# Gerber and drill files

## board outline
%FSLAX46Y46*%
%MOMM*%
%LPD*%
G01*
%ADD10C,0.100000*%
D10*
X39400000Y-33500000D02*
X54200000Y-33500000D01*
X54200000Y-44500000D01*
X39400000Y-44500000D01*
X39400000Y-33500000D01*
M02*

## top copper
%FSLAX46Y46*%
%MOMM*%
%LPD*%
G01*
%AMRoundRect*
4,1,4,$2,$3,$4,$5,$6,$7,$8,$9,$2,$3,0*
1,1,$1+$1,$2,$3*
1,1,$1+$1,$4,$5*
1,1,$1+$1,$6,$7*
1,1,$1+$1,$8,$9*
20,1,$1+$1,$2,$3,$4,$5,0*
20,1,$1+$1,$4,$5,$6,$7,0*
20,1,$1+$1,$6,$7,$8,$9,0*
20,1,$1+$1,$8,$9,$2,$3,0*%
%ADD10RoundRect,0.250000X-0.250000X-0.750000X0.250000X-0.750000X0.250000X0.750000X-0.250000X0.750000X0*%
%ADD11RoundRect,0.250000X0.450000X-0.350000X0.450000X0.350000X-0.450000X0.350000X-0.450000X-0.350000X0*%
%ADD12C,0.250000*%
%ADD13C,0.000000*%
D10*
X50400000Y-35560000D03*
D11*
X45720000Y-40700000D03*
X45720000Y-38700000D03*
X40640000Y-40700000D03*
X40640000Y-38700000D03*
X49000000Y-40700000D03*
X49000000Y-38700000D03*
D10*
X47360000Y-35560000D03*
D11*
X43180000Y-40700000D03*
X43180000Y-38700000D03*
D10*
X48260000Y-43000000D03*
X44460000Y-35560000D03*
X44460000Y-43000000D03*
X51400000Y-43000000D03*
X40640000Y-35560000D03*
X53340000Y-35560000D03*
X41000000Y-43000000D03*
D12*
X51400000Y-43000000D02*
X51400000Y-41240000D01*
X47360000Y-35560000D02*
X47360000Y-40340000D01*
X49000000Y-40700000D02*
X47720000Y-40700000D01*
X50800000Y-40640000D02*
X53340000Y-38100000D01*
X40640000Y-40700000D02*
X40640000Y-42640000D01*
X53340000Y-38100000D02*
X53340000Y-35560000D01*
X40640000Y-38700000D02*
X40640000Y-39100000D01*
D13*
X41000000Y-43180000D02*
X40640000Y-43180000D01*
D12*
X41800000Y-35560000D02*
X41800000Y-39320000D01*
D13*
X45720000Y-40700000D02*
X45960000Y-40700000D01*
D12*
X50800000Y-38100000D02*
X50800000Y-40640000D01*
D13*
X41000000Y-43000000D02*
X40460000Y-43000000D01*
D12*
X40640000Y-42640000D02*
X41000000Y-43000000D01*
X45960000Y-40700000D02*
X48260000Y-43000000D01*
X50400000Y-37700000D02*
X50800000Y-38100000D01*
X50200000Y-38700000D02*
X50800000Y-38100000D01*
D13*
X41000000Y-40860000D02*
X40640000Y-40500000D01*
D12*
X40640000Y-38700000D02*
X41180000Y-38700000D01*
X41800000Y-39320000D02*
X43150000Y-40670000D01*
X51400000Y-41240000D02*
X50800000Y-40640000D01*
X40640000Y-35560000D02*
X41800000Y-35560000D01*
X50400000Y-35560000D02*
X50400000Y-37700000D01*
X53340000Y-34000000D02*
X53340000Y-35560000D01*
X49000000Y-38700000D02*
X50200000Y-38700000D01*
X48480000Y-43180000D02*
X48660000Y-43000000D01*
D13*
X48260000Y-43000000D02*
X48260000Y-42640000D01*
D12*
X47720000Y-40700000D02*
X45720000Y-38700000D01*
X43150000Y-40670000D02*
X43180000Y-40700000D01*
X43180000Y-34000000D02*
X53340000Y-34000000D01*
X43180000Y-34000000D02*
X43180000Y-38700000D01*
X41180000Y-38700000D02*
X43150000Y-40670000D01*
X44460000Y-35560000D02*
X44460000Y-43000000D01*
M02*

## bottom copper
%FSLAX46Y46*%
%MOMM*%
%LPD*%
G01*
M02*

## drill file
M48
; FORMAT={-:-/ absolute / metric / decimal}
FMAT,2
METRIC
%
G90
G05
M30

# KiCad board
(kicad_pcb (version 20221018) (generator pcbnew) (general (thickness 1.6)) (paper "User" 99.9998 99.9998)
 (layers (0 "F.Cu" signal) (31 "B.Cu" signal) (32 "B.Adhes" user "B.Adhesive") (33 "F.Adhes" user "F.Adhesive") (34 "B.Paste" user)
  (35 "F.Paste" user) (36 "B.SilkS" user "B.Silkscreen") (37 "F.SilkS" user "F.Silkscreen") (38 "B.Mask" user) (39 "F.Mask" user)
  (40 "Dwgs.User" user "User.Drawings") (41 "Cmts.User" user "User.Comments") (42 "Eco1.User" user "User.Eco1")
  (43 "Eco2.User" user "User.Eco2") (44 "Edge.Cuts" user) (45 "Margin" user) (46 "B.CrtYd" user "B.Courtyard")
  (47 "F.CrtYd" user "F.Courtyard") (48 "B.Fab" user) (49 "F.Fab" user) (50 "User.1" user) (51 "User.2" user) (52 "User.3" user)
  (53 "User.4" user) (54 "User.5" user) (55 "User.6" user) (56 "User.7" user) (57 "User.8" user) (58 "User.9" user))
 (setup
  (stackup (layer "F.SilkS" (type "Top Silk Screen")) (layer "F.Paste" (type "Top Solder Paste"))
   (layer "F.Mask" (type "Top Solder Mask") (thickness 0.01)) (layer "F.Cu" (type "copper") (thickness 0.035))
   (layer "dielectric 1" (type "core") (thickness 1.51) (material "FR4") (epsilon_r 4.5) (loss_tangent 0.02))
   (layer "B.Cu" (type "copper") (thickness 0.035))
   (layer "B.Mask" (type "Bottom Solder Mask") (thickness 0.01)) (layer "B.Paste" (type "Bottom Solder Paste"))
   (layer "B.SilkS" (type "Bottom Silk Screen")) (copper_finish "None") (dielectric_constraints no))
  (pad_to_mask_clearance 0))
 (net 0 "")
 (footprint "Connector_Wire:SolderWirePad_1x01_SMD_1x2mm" (layer "F.Cu") (at 50.4 35.56)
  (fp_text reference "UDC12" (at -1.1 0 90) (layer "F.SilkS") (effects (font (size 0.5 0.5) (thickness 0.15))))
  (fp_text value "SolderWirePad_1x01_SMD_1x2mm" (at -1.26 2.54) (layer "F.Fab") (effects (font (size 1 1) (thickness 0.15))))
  (pad "1" smd roundrect (at 0 0) (size 1 2) (layers "F.Cu" "F.Paste" "F.Mask") (roundrect_rratio 0.25)))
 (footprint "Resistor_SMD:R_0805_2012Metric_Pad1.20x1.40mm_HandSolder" (layer "F.Cu") (at 45.72 39.7 90)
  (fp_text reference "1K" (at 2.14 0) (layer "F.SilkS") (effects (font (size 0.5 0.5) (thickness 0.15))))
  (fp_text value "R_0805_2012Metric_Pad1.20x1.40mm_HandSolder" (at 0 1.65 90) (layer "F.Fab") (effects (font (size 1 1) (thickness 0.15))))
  (pad "1" smd roundrect (at -1 0 90) (size 1.2 1.4) (layers "F.Cu" "F.Paste" "F.Mask") (roundrect_rratio 0.2083333333))
  (pad "2" smd roundrect (at 1 0 90) (size 1.2 1.4) (layers "F.Cu" "F.Paste" "F.Mask") (roundrect_rratio 0.2083333333)))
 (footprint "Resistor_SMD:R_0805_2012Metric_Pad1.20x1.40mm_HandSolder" (layer "F.Cu") (at 40.64 39.7 90)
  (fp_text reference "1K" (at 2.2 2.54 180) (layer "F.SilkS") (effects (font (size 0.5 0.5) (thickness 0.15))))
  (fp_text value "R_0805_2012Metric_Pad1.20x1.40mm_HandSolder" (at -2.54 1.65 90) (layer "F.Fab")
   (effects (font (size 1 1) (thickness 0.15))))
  (pad "1" smd roundrect (at -1 0 90) (size 1.2 1.4) (layers "F.Cu" "F.Paste" "F.Mask") (roundrect_rratio 0.2083333333))
  (pad "2" smd roundrect (at 1 0 90) (size 1.2 1.4) (layers "F.Cu" "F.Paste" "F.Mask") (roundrect_rratio 0.2083333333)))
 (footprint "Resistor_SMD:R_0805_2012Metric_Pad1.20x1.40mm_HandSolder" (layer "F.Cu") (at 49 39.7 90)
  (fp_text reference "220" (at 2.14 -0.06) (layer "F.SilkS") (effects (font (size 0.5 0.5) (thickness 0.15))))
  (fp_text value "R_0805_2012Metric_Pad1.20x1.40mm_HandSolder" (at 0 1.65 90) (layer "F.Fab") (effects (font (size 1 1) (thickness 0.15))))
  (pad "1" smd roundrect (at -1 0 90) (size 1.2 1.4) (layers "F.Cu" "F.Paste" "F.Mask") (roundrect_rratio 0.2083333333))
  (pad "2" smd roundrect (at 1 0 90) (size 1.2 1.4) (layers "F.Cu" "F.Paste" "F.Mask") (roundrect_rratio 0.2083333333)))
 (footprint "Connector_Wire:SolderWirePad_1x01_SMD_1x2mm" (layer "F.Cu") (at 47.36 35.56)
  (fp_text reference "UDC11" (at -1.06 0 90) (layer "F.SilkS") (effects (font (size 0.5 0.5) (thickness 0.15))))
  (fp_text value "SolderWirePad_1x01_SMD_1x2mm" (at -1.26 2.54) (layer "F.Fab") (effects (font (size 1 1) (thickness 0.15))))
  (pad "1" smd roundrect (at 0 0) (size 1 2) (layers "F.Cu" "F.Paste" "F.Mask") (roundrect_rratio 0.25)))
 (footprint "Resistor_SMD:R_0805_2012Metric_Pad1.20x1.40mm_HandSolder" (layer "F.Cu") (at 43.18 39.7 90)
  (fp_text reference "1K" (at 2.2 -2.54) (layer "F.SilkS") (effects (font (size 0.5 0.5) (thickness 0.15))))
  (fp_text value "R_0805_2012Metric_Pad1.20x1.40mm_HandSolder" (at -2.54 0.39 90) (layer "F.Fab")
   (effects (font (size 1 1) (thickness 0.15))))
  (pad "1" smd roundrect (at -1 0 90) (size 1.2 1.4) (layers "F.Cu" "F.Paste" "F.Mask") (roundrect_rratio 0.2083333333))
  (pad "2" smd roundrect (at 1 0 90) (size 1.2 1.4) (layers "F.Cu" "F.Paste" "F.Mask") (roundrect_rratio 0.2083333333)))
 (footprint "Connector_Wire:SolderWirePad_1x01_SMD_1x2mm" (layer "F.Cu") (at 48.26 43)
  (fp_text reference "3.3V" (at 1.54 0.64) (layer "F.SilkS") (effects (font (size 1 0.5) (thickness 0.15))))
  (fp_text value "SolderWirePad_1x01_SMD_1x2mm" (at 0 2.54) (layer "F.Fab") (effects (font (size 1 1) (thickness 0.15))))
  (pad "1" smd roundrect (at 0 0) (size 1 2) (layers "F.Cu" "F.Paste" "F.Mask") (roundrect_rratio 0.25)))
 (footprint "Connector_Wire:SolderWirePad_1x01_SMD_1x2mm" (layer "F.Cu") (at 44.46 35.56)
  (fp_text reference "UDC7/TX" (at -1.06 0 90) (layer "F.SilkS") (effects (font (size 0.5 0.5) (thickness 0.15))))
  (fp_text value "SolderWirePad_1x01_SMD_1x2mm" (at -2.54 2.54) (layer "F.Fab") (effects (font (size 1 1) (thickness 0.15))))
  (pad "1" smd roundrect (at 0 0) (size 1 2) (layers "F.Cu" "F.Paste" "F.Mask") (roundrect_rratio 0.25)))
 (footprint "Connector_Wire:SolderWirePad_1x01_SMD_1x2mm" (layer "F.Cu") (at 44.46 43)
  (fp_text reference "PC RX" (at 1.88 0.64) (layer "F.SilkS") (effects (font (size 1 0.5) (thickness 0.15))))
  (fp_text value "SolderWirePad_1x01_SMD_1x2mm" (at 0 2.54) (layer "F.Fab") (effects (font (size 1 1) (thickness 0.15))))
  (pad "1" smd roundrect (at 0 0) (size 1 2) (layers "F.Cu" "F.Paste" "F.Mask") (roundrect_rratio 0.25)))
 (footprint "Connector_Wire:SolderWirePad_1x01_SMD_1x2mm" (layer "F.Cu") (at 51.4 43)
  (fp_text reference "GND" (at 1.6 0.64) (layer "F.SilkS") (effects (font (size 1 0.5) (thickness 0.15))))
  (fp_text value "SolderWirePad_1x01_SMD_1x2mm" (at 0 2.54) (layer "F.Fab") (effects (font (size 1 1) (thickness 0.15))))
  (pad "1" smd roundrect (at 0 0) (size 1 2) (layers "F.Cu" "F.Paste" "F.Mask") (roundrect_rratio 0.25)))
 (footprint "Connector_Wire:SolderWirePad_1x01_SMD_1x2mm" (layer "F.Cu") (at 40.64 35.56)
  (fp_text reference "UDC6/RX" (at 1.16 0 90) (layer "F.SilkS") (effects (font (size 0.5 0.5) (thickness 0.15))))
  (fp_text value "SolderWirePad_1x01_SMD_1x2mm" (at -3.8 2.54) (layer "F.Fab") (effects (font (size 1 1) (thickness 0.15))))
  (pad "1" smd roundrect (at 0 0) (size 1 2) (layers "F.Cu" "F.Paste" "F.Mask") (roundrect_rratio 0.25)))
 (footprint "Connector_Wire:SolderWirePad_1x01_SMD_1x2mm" (layer "F.Cu") (at 53.34 35.56)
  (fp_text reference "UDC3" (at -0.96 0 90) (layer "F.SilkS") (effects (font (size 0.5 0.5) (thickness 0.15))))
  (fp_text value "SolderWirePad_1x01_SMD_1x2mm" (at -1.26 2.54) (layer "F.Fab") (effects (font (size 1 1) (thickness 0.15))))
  (pad "1" smd roundrect (at 0 0) (size 1 2) (layers "F.Cu" "F.Paste" "F.Mask") (roundrect_rratio 0.25)))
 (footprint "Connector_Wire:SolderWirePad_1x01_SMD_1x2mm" (layer "F.Cu") (at 41 43)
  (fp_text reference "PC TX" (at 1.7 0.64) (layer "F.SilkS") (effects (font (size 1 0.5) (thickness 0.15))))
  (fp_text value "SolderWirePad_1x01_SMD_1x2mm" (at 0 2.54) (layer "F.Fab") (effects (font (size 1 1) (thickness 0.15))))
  (pad "1" smd roundrect (at 0 0) (size 1 2) (layers "F.Cu" "F.Paste" "F.Mask") (roundrect_rratio 0.25)))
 (gr_rect (start 39.4 33.5) (end 54.2 44.5) (stroke (width 0.1) (type default)) (fill none) (layer "Edge.Cuts"))
 (segment (start 51.4 43) (end 51.4 41.24) (width 0.25) (layer "F.Cu") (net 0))
 (segment (start 47.36 35.56) (end 47.36 40.34) (width 0.25) (layer "F.Cu") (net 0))
 (segment (start 49 40.7) (end 47.72 40.7) (width 0.25) (layer "F.Cu") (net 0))
 (segment (start 50.8 40.64) (end 53.34 38.1) (width 0.25) (layer "F.Cu") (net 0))
 (segment (start 40.64 40.7) (end 40.64 42.64) (width 0.25) (layer "F.Cu") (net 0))
 (segment (start 53.34 38.1) (end 53.34 35.56) (width 0.25) (layer "F.Cu") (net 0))
 (segment (start 40.64 38.7) (end 40.64 39.1) (width 0.25) (layer "F.Cu") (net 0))
 (segment (start 41 43.18) (end 40.64 43.18) (width 0) (layer "F.Cu") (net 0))
 (segment (start 41.8 35.56) (end 41.8 39.32) (width 0.25) (layer "F.Cu") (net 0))
 (segment (start 45.72 40.7) (end 45.96 40.7) (width 0) (layer "F.Cu") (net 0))
 (segment (start 50.8 38.1) (end 50.8 40.64) (width 0.25) (layer "F.Cu") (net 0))
 (segment (start 41 43) (end 40.46 43) (width 0) (layer "F.Cu") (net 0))
 (segment (start 40.64 42.64) (end 41 43) (width 0.25) (layer "F.Cu") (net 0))
 (segment (start 45.96 40.7) (end 48.26 43) (width 0.25) (layer "F.Cu") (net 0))
 (segment (start 50.4 37.7) (end 50.8 38.1) (width 0.25) (layer "F.Cu") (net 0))
 (segment (start 50.2 38.7) (end 50.8 38.1) (width 0.25) (layer "F.Cu") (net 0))
 (segment (start 41 40.86) (end 40.64 40.5) (width 0) (layer "F.Cu") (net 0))
 (segment (start 40.64 38.7) (end 41.18 38.7) (width 0.25) (layer "F.Cu") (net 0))
 (segment (start 41.8 39.32) (end 43.15 40.67) (width 0.25) (layer "F.Cu") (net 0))
 (segment (start 51.4 41.24) (end 50.8 40.64) (width 0.25) (layer "F.Cu") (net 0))
 (segment (start 40.64 35.56) (end 41.8 35.56) (width 0.25) (layer "F.Cu") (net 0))
 (segment (start 50.4 35.56) (end 50.4 37.7) (width 0.25) (layer "F.Cu") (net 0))
 (segment (start 53.34 34) (end 53.34 35.56) (width 0.25) (layer "F.Cu") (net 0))
 (segment (start 49 38.7) (end 50.2 38.7) (width 0.25) (layer "F.Cu") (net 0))
 (segment (start 48.48 43.18) (end 48.66 43) (width 0.25) (layer "F.Cu") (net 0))
 (segment (start 48.26 43) (end 48.26 42.64) (width 0) (layer "F.Cu") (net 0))
 (segment (start 47.72 40.7) (end 45.72 38.7) (width 0.25) (layer "F.Cu") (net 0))
 (segment (start 43.15 40.67) (end 43.18 40.7) (width 0.25) (layer "F.Cu") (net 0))
 (segment (start 43.18 34) (end 53.34 34) (width 0.25) (layer "F.Cu") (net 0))
 (segment (start 43.18 34) (end 43.18 38.7) (width 0.25) (layer "F.Cu") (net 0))
 (segment (start 41.18 38.7) (end 43.15 40.67) (width 0.25) (layer "F.Cu") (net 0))
 (segment (start 44.46 35.56) (end 44.46 43) (width 0.25) (layer "F.Cu") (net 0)))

